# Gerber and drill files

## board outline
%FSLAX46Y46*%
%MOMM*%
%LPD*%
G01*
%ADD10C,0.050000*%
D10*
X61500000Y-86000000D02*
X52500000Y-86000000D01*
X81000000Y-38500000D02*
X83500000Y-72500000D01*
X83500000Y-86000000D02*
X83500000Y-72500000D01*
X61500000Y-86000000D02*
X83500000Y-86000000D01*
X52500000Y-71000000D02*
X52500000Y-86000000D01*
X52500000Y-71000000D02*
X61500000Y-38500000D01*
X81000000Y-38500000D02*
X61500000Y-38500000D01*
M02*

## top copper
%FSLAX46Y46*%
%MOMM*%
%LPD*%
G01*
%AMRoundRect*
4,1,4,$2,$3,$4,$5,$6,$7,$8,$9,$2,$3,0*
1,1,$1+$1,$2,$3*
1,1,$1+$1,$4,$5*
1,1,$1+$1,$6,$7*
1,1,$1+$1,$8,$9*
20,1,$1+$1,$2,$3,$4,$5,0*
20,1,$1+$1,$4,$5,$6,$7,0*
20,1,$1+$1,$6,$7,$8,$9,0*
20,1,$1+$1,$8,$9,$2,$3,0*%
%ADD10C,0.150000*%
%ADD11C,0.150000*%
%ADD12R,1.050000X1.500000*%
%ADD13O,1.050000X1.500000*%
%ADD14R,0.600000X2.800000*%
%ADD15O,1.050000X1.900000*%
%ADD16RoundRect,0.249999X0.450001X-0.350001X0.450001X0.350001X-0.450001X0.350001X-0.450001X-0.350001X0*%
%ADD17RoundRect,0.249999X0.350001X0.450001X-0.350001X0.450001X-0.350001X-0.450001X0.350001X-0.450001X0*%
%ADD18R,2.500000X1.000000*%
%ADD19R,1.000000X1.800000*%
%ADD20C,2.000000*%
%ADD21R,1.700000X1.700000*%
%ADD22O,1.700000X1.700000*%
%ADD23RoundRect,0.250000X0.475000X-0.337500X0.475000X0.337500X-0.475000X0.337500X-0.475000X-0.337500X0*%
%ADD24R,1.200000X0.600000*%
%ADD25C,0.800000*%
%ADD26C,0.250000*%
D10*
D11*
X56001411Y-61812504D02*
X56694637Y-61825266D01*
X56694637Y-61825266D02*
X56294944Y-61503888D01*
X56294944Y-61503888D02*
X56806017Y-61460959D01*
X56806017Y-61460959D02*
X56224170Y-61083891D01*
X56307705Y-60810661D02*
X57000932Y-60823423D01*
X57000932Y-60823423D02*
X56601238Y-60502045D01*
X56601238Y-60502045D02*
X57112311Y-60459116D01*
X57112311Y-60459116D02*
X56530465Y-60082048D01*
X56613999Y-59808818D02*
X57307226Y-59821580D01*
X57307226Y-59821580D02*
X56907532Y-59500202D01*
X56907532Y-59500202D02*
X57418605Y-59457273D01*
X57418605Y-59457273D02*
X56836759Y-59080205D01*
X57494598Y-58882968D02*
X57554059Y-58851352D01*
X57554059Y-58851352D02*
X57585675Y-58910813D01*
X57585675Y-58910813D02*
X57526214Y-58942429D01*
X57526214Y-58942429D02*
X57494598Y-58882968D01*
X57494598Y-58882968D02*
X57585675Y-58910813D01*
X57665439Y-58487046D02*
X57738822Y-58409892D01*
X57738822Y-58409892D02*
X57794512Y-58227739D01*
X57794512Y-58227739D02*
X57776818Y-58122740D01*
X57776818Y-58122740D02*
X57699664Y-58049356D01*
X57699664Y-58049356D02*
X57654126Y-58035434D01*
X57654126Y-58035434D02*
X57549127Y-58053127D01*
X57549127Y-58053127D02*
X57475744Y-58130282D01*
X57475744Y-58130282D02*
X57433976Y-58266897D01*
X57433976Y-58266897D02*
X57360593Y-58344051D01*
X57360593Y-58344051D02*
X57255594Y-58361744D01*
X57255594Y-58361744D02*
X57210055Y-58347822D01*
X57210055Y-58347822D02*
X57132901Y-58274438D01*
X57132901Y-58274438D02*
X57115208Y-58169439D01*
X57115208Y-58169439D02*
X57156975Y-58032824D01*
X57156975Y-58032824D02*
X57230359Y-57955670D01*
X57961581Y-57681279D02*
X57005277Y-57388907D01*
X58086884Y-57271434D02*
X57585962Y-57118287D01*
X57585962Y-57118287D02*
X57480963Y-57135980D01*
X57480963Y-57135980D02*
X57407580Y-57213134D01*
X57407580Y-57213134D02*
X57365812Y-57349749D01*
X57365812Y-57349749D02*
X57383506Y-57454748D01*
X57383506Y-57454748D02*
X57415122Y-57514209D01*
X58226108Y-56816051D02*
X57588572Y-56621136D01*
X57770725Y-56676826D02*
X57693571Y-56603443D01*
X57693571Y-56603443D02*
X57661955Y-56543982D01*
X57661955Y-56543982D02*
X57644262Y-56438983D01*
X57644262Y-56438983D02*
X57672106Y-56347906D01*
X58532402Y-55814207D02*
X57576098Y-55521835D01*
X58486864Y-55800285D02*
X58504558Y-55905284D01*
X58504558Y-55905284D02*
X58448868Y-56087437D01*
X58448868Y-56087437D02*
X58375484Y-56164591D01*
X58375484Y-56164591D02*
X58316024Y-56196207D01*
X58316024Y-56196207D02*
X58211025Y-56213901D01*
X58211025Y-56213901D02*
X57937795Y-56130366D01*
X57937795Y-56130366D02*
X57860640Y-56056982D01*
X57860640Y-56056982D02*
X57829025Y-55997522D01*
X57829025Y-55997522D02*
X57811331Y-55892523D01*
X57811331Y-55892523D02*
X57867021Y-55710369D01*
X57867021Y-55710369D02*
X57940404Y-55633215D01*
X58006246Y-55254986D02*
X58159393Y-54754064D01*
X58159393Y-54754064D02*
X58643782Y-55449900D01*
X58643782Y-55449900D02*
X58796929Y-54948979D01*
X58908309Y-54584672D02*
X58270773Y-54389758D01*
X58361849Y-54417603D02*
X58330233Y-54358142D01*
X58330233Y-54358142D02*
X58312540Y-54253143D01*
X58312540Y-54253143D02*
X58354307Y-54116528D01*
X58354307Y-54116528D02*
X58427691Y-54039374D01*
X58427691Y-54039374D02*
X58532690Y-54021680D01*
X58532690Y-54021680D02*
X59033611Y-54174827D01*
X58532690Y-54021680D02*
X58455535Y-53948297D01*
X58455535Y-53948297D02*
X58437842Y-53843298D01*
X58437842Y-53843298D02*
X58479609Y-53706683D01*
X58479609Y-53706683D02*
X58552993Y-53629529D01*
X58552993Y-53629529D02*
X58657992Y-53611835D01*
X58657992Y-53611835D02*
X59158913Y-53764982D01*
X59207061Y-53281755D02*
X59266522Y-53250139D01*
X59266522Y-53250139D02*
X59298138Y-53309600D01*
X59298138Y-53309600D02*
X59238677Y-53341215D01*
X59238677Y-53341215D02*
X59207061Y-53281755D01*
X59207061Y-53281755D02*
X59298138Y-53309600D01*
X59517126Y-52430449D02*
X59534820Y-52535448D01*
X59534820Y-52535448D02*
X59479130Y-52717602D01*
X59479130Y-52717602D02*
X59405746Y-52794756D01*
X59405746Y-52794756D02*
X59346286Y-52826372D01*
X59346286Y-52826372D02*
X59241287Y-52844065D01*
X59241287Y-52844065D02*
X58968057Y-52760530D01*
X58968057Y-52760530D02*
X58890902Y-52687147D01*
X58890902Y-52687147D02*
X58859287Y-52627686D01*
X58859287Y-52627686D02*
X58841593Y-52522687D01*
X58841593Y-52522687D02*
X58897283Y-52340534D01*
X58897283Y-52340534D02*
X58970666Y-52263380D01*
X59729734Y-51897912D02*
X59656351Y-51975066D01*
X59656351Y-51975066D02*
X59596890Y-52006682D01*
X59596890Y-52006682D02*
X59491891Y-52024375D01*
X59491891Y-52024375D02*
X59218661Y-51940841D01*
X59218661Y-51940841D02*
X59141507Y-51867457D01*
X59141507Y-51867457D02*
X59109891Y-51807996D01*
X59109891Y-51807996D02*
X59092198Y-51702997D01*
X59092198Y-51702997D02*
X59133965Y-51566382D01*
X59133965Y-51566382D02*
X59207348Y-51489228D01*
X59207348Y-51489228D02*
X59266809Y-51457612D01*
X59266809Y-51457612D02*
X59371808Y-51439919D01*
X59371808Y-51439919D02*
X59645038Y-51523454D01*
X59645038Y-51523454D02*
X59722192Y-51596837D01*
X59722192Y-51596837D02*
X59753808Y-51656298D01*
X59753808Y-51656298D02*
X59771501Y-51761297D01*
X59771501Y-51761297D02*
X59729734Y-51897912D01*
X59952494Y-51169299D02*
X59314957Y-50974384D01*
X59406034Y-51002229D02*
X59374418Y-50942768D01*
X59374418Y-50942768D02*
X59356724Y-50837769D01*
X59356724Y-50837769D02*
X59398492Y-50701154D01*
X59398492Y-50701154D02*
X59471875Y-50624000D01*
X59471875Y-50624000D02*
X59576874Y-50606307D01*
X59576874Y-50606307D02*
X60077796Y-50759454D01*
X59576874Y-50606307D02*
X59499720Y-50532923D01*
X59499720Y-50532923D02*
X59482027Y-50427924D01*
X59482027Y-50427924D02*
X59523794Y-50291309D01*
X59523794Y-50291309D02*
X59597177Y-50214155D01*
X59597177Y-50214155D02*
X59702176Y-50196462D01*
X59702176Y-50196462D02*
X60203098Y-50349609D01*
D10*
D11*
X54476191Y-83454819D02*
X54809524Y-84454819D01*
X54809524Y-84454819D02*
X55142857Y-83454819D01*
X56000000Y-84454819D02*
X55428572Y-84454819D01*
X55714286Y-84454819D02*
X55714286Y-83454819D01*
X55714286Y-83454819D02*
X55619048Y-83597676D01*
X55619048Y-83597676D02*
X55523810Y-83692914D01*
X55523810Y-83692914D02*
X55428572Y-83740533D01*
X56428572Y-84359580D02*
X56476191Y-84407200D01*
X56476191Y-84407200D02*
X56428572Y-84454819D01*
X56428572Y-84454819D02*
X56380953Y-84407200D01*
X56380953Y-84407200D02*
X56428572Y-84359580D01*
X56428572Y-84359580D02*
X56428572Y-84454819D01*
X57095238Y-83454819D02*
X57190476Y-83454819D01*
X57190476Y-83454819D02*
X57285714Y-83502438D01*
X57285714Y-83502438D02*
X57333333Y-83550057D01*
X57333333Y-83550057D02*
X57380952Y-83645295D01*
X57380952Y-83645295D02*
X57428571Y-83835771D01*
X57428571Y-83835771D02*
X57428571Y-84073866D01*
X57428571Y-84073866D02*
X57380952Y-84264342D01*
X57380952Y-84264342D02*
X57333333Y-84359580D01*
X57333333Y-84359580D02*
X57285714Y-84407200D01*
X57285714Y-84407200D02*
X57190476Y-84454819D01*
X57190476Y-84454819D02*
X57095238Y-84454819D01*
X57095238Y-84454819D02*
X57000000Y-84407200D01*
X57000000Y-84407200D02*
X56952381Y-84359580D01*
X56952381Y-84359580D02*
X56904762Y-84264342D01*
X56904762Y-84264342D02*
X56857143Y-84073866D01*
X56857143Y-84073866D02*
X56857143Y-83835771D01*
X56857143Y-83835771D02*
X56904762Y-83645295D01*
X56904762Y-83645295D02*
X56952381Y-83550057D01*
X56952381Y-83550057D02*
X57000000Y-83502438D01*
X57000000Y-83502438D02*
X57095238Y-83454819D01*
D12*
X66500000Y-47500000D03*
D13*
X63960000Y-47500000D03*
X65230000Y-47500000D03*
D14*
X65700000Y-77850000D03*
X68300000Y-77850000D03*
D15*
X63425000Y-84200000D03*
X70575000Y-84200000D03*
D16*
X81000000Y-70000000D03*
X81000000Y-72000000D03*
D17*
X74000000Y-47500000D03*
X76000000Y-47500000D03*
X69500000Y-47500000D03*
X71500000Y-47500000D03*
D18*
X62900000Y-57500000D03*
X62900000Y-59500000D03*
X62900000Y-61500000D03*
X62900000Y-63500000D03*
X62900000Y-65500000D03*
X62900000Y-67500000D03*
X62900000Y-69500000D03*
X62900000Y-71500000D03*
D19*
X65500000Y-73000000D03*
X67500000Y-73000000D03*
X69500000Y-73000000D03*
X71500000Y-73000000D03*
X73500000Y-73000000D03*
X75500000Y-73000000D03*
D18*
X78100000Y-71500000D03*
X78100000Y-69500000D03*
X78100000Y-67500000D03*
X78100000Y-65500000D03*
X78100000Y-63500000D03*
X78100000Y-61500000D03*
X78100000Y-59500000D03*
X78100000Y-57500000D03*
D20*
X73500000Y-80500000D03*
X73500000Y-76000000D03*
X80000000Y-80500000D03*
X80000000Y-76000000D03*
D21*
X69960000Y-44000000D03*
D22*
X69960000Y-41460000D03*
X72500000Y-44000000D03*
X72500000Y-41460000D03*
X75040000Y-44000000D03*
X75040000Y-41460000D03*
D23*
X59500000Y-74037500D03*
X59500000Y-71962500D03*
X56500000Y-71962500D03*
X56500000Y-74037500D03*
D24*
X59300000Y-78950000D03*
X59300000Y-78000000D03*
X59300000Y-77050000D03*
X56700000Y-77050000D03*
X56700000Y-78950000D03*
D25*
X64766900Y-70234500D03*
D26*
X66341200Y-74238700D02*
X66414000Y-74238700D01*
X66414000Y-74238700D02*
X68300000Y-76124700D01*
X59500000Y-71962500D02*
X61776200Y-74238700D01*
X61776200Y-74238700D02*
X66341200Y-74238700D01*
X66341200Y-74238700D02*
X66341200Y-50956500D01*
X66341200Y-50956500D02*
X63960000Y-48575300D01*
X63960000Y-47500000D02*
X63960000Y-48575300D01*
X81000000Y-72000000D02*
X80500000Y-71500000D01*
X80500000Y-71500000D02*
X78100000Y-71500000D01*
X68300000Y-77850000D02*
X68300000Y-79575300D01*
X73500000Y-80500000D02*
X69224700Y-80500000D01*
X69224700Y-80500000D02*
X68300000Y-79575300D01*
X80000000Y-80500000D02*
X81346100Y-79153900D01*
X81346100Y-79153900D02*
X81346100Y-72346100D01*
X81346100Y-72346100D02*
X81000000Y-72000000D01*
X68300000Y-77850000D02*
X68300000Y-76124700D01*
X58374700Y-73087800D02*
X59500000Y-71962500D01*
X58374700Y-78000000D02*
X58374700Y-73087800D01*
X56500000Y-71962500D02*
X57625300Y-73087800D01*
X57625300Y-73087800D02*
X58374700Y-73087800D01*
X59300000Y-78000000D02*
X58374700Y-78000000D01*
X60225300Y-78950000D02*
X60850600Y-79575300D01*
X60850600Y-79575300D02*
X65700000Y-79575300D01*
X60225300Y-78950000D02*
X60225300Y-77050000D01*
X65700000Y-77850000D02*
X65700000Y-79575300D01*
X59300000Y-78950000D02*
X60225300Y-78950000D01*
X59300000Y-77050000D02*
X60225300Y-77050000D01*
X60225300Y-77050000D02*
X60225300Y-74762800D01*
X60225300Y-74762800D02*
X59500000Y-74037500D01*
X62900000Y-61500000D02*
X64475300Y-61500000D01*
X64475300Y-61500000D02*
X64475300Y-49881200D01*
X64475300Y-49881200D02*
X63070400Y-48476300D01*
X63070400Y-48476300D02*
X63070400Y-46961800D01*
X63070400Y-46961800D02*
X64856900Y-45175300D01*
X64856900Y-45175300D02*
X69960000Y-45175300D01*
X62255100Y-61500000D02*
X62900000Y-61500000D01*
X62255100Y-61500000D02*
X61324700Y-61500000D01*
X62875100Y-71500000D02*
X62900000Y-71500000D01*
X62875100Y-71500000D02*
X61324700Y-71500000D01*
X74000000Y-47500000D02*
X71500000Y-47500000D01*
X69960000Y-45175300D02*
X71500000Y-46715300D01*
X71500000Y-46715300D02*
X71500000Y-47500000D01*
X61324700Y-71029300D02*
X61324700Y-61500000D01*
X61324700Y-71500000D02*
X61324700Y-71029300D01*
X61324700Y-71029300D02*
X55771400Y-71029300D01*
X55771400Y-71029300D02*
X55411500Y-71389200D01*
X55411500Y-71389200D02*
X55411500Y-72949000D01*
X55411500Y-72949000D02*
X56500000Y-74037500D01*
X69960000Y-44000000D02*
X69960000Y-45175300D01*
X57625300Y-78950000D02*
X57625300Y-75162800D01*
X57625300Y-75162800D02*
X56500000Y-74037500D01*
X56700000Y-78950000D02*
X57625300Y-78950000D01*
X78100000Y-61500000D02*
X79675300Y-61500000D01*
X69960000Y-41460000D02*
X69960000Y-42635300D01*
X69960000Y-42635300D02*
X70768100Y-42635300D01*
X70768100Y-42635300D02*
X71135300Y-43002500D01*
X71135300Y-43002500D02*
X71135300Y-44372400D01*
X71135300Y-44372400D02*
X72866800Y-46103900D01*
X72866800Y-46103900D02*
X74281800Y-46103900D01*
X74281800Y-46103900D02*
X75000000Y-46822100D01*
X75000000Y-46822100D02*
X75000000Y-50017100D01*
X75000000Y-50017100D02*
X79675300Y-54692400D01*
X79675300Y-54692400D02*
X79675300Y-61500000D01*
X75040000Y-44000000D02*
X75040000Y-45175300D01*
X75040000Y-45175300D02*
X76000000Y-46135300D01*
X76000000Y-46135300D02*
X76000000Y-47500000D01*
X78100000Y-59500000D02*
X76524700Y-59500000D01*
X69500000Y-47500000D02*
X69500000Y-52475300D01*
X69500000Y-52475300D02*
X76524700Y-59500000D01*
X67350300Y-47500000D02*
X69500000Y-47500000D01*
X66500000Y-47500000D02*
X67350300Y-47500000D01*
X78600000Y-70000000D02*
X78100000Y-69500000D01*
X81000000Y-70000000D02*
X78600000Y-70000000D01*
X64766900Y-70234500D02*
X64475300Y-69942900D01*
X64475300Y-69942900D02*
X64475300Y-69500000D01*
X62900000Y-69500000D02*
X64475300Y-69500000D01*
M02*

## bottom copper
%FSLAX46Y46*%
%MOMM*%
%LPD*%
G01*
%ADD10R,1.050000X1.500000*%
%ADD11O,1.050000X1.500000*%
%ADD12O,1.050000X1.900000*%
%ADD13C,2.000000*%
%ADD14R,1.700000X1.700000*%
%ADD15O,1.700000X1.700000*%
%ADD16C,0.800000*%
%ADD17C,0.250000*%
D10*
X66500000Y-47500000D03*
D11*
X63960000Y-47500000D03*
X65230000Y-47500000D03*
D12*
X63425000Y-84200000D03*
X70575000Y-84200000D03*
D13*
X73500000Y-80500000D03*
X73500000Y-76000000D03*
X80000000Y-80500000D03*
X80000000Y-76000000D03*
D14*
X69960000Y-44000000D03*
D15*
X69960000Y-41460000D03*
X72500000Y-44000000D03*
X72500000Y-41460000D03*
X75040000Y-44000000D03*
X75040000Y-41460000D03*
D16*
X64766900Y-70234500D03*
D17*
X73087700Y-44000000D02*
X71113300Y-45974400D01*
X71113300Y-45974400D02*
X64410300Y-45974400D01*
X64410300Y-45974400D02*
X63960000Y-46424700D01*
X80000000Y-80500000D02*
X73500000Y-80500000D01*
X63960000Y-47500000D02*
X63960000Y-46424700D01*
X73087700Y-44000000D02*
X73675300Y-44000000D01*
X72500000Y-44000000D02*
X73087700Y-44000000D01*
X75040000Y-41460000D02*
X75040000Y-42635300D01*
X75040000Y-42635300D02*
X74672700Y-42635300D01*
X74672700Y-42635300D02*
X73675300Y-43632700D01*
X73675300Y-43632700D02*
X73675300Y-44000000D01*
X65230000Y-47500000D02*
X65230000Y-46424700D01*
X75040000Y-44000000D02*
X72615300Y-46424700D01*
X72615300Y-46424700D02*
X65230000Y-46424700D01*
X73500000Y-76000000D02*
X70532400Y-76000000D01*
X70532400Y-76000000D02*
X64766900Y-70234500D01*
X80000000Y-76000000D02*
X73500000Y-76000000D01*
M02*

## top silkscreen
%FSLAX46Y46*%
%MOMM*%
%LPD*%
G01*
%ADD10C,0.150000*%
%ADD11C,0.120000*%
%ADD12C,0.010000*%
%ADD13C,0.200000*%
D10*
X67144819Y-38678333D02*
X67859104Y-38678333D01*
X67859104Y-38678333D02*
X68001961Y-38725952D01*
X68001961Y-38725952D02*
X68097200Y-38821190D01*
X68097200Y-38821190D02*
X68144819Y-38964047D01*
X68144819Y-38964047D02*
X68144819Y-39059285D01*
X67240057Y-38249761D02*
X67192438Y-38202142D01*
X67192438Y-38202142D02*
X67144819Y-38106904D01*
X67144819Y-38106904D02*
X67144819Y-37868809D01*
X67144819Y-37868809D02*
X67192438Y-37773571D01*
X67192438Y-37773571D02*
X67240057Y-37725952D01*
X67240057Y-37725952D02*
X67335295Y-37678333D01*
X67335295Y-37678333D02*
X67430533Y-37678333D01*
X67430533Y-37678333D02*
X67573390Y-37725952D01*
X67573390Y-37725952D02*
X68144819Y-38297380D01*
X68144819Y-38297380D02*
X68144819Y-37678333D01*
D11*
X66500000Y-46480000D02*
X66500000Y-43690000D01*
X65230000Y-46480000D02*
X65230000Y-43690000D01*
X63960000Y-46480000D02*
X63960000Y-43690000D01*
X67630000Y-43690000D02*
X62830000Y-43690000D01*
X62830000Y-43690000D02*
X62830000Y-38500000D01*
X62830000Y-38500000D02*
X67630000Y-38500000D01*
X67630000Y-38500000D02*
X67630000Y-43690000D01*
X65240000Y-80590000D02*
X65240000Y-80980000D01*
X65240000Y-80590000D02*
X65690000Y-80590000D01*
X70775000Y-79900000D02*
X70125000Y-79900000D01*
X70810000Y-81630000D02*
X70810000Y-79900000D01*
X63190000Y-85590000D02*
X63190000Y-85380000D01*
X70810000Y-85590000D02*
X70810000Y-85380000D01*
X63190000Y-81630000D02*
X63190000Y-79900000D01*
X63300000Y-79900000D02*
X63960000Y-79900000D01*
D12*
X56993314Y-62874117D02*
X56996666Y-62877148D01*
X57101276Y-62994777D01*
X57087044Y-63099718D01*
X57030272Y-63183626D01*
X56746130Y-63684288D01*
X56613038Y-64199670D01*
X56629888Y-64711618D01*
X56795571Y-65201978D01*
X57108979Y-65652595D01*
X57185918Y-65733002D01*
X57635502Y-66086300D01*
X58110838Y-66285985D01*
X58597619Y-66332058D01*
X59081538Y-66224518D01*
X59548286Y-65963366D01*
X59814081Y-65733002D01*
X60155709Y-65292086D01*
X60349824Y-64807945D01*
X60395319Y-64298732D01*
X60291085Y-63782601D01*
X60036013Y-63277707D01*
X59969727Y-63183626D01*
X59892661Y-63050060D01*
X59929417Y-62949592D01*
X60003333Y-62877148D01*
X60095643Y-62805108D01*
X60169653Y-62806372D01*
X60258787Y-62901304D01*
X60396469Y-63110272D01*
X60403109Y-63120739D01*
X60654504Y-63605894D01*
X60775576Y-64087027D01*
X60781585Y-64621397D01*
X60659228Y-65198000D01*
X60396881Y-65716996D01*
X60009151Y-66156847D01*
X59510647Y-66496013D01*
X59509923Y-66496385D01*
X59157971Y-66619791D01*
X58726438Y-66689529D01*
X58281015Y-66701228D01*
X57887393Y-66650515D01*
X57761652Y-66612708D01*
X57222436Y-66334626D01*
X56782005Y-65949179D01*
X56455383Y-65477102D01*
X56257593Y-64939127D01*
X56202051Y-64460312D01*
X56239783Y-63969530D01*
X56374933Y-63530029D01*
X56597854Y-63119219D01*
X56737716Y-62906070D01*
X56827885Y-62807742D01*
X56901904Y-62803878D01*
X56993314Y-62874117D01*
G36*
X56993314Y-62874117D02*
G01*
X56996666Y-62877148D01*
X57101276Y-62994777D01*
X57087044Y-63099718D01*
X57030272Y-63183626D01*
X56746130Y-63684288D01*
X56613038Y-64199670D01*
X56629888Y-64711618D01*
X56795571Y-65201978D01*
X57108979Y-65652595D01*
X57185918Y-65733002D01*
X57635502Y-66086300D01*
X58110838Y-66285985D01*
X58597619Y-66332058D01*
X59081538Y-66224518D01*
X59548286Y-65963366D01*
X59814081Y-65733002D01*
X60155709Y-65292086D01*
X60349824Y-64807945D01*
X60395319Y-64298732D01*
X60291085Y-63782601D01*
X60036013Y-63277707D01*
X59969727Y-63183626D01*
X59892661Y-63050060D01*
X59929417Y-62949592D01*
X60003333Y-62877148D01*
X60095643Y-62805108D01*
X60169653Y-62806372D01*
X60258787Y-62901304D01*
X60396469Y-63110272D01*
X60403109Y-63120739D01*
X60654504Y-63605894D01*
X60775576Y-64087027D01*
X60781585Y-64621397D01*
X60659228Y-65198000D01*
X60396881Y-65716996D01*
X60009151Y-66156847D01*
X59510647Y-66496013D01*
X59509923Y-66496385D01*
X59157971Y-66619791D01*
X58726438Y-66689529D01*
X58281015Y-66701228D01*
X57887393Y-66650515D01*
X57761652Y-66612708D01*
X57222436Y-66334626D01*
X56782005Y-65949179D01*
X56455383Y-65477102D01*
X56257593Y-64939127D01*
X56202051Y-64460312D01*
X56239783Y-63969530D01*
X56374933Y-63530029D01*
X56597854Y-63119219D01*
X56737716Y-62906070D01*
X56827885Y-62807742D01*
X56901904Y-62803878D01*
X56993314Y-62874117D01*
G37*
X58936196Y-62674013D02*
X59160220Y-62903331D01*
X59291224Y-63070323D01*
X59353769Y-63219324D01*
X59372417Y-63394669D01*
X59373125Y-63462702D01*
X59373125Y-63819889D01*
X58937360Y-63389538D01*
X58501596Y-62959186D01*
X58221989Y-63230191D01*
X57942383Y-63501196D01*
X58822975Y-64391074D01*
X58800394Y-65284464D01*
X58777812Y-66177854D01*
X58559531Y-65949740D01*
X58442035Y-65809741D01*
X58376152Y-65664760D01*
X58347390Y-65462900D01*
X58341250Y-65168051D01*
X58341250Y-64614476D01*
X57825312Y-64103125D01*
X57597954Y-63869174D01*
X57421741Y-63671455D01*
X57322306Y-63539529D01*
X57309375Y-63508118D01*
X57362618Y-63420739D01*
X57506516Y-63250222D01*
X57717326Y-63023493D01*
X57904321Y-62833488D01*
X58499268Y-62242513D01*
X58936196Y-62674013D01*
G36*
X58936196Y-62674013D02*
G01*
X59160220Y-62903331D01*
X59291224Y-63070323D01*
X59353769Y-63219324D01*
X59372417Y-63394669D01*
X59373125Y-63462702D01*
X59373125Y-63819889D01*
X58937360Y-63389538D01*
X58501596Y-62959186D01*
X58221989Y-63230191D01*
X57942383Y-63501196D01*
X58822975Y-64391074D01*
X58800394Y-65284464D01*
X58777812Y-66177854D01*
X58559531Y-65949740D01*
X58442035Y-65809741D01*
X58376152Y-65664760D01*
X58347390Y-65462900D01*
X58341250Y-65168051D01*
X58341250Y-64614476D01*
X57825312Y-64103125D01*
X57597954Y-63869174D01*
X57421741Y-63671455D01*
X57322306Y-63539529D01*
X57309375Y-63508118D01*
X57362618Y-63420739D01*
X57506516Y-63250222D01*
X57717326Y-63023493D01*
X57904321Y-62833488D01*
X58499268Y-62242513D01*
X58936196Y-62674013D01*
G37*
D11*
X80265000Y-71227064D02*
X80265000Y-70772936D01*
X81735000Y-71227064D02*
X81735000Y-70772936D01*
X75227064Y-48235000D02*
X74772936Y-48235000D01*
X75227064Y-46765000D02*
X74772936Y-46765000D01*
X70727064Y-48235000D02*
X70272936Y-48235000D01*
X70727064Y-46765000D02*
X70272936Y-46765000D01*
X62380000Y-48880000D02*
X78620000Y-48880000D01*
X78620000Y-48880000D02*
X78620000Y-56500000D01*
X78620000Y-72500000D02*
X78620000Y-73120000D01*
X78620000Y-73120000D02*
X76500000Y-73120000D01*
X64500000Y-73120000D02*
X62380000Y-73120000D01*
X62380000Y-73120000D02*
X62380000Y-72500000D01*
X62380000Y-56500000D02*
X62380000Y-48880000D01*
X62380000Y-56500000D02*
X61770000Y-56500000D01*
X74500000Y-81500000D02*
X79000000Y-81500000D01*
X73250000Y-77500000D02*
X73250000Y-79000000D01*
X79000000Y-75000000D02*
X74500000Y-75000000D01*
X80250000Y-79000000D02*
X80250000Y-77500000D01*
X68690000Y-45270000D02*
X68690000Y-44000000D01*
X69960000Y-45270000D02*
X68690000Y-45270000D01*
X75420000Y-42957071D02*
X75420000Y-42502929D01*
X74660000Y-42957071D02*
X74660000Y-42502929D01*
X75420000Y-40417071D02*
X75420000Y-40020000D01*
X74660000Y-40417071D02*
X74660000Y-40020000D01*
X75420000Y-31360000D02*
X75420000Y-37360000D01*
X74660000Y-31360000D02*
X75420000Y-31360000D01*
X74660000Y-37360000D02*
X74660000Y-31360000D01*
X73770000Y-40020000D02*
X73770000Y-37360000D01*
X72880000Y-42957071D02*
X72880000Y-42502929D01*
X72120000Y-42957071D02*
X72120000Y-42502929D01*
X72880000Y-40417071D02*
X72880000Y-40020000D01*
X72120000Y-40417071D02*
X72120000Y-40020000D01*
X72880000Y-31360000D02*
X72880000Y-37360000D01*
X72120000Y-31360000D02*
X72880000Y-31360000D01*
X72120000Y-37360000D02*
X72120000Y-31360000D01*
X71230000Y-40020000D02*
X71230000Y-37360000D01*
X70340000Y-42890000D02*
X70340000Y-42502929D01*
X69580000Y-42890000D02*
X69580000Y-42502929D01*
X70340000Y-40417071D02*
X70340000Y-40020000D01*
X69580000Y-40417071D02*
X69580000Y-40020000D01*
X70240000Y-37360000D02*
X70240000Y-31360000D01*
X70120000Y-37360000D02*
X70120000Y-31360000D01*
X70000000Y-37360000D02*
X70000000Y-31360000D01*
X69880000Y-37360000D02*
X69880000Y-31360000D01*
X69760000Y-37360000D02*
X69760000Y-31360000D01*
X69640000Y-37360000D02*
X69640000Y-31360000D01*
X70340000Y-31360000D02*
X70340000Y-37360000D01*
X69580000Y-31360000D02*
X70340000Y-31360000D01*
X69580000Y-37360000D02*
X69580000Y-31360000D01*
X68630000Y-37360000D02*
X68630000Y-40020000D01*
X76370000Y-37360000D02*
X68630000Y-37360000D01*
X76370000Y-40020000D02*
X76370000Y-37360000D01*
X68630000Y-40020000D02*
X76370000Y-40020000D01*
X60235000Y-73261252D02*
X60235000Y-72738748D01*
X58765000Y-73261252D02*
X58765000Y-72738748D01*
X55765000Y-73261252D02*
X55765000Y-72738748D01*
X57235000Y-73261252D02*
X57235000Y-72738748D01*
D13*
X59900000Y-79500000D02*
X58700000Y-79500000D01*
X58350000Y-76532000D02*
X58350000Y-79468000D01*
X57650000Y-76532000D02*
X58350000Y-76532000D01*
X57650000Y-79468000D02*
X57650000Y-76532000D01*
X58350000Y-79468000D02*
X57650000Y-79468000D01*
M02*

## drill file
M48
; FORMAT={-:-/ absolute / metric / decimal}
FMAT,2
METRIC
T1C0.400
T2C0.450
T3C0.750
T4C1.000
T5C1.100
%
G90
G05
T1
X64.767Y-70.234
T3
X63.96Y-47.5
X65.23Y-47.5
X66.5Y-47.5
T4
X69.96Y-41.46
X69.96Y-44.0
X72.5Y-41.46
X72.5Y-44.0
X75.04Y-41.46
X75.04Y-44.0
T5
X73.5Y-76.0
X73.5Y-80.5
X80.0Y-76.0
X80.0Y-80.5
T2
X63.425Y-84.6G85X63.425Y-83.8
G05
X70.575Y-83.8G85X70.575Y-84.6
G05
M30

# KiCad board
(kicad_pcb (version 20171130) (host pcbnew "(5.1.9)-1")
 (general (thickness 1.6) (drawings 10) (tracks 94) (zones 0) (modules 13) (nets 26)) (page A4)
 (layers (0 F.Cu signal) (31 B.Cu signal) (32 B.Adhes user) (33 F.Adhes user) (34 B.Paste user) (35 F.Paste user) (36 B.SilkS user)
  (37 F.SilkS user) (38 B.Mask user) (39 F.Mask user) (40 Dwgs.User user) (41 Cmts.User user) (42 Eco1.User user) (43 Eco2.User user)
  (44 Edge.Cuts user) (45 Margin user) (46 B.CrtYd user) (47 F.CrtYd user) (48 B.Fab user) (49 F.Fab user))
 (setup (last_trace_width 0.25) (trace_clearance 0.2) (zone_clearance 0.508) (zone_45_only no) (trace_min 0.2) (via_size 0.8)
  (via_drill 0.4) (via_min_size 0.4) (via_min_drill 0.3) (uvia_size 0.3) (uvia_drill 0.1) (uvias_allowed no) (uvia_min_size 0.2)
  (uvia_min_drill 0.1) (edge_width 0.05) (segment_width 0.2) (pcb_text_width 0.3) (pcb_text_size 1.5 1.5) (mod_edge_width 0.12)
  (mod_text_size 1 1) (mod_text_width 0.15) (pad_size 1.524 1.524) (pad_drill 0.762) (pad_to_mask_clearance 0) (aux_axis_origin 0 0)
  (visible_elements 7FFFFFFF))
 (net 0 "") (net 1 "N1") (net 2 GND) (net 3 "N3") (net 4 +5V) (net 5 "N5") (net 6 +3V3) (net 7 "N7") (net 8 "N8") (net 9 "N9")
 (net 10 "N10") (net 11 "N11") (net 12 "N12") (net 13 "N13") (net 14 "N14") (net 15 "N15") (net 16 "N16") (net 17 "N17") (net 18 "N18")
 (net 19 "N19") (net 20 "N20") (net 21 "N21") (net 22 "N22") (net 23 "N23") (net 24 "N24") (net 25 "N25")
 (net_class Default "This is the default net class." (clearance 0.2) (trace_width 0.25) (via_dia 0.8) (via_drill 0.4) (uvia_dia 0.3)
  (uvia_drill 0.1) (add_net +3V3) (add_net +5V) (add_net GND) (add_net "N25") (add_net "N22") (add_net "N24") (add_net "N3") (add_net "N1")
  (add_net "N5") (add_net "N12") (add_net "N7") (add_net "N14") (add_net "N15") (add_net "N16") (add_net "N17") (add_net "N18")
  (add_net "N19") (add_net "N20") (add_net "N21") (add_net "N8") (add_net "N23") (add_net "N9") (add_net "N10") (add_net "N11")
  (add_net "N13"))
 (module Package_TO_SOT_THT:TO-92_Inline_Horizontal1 (layer F.Cu) (at 66.5 47.5 180)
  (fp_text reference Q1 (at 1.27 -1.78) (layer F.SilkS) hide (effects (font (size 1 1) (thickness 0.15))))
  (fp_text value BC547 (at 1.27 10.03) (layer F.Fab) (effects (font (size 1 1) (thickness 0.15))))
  (fp_line (start 0 1.02) (end 0 3.81) (layer F.SilkS) (width 0.12))
  (fp_line (start 1.27 1.02) (end 1.27 3.81) (layer F.SilkS) (width 0.12))
  (fp_line (start 2.54 1.02) (end 2.54 3.81) (layer F.SilkS) (width 0.12))
  (fp_line (start -1.13 3.81) (end 3.67 3.81) (layer F.SilkS) (width 0.12))
  (fp_line (start 3.67 3.81) (end 3.67 9) (layer F.SilkS) (width 0.12))
  (fp_line (start 3.67 9) (end -1.13 9) (layer F.SilkS) (width 0.12))
  (fp_line (start -1.13 9) (end -1.13 3.81) (layer F.SilkS) (width 0.12))
  (pad 1 thru_hole rect (at 0 0 180) (size 1.05 1.5) (drill 0.75) (layers *.Cu *.Mask) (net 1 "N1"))
  (pad 3 thru_hole oval (at 2.54 0 180) (size 1.05 1.5) (drill 0.75) (layers *.Cu *.Mask) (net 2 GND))
  (pad 2 thru_hole oval (at 1.27 0 180) (size 1.05 1.5) (drill 0.75) (layers *.Cu *.Mask) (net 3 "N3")))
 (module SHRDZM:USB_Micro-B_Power (layer F.Cu) (at 67 83)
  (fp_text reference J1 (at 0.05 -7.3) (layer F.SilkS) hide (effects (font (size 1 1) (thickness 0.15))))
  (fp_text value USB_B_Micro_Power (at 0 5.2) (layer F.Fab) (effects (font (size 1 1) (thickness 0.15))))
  (fp_line (start -1.76 -2.41) (end -1.76 -2.02) (layer F.SilkS) (width 0.12))
  (fp_line (start -1.76 -2.41) (end -1.31 -2.41) (layer F.SilkS) (width 0.12))
  (fp_line (start 3.775 -3.1) (end 3.125 -3.1) (layer F.SilkS) (width 0.12))
  (fp_line (start 3.81 -1.37) (end 3.81 -3.1) (layer F.SilkS) (width 0.12))
  (fp_line (start -3.81 2.59) (end -3.81 2.38) (layer F.SilkS) (width 0.12))
  (fp_line (start 3.81 2.59) (end 3.81 2.38) (layer F.SilkS) (width 0.12))
  (fp_line (start -3.81 -1.37) (end -3.81 -3.1) (layer F.SilkS) (width 0.12))
  (fp_line (start -3.7 -3.1) (end -3.04 -3.1) (layer F.SilkS) (width 0.12))
  (pad 1 smd rect (at -1.3 -5.15) (size 0.6 2.8) (layers F.Cu F.Paste F.Mask) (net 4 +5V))
  (pad 5 smd rect (at 1.3 -5.15) (size 0.6 2.8) (layers F.Cu F.Paste F.Mask) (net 2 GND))
  (pad "" thru_hole oval (at -3.575 1.2 180) (size 1.05 1.9) (drill oval 0.45 1.25) (layers *.Cu *.Mask))
  (pad "" thru_hole oval (at 3.575 1.2) (size 1.05 1.9) (drill oval 0.45 1.25) (layers *.Cu *.Mask)))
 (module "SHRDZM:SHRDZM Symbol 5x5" (layer F.Cu) (at 58.5 64.5)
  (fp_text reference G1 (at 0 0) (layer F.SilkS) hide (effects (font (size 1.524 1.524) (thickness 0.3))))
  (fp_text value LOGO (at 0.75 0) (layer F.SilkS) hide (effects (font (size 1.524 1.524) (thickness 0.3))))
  (fp_poly
   (pts (xy -1.506686 -1.625883) (xy -1.503334 -1.622852) (xy -1.398724 -1.505223) (xy -1.412956 -1.400282) (xy -1.469728 -1.316374)
    (xy -1.75387 -0.815712) (xy -1.886962 -0.30033) (xy -1.870112 0.211618) (xy -1.704429 0.701978) (xy -1.391021 1.152595)
    (xy -1.314082 1.233002) (xy -0.864498 1.5863) (xy -0.389162 1.785985) (xy 0.097619 1.832058) (xy 0.581538 1.724518)
    (xy 1.048286 1.463366) (xy 1.314081 1.233002) (xy 1.655709 0.792086) (xy 1.849824 0.307945) (xy 1.895319 -0.201268)
    (xy 1.791085 -0.717399) (xy 1.536013 -1.222293) (xy 1.469727 -1.316374) (xy 1.392661 -1.44994) (xy 1.429417 -1.550408)
    (xy 1.503333 -1.622852) (xy 1.595643 -1.694892) (xy 1.669653 -1.693628) (xy 1.758787 -1.598696) (xy 1.896469 -1.389728)
    (xy 1.903109 -1.379261) (xy 2.154504 -0.894106) (xy 2.275576 -0.412973) (xy 2.281585 0.121397) (xy 2.159228 0.698)
    (xy 1.896881 1.216996) (xy 1.509151 1.656847) (xy 1.010647 1.996013) (xy 1.009923 1.996385) (xy 0.657971 2.119791)
    (xy 0.226438 2.189529) (xy -0.218985 2.201228) (xy -0.612607 2.150515) (xy -0.738348 2.112708) (xy -1.277564 1.834626)
    (xy -1.717995 1.449179) (xy -2.044617 0.977102) (xy -2.242407 0.439127) (xy -2.297949 -0.039688) (xy -2.260217 -0.53047)
    (xy -2.125067 -0.969971) (xy -1.902146 -1.380781) (xy -1.762284 -1.59393) (xy -1.672115 -1.692258) (xy -1.598096 -1.696122)
    (xy -1.506686 -1.625883))
   (layer F.SilkS) (width 0.01))
  (fp_poly
   (pts (xy 0.436196 -1.825987) (xy 0.66022 -1.596669) (xy 0.791224 -1.429677) (xy 0.853769 -1.280676) (xy 0.872417 -1.105331)
    (xy 0.873125 -1.037298) (xy 0.873125 -0.680111) (xy 0.43736 -1.110462) (xy 0.001596 -1.540814) (xy -0.278011 -1.269809)
    (xy -0.557617 -0.998804) (xy 0.322975 -0.108926) (xy 0.300394 0.784464) (xy 0.277812 1.677854) (xy 0.059531 1.44974)
    (xy -0.057965 1.309741) (xy -0.123848 1.16476) (xy -0.15261 0.9629) (xy -0.15875 0.668051) (xy -0.15875 0.114476)
    (xy -0.674688 -0.396875) (xy -0.902046 -0.630826) (xy -1.078259 -0.828545) (xy -1.177694 -0.960471) (xy -1.190625 -0.991882)
    (xy -1.137382 -1.079261) (xy -0.993484 -1.249778) (xy -0.782674 -1.476507) (xy -0.595679 -1.666512) (xy -0.000732 -2.257487)
    (xy 0.436196 -1.825987))
   (layer F.SilkS) (width 0.01)))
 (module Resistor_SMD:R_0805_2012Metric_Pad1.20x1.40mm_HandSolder (layer F.Cu) (at 81 71 90)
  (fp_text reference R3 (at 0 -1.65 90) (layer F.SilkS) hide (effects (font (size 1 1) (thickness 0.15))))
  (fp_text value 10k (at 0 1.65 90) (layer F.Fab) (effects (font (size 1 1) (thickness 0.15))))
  (fp_line (start -0.227064 -0.735) (end 0.227064 -0.735) (layer F.SilkS) (width 0.12))
  (fp_line (start -0.227064 0.735) (end 0.227064 0.735) (layer F.SilkS) (width 0.12))
  (pad 2 smd roundrect (at 1 0 90) (size 1.2 1.4) (layers F.Cu F.Paste F.Mask) (roundrect_rratio 0.2083325) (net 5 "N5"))
  (pad 1 smd roundrect (at -1 0 90) (size 1.2 1.4) (layers F.Cu F.Paste F.Mask) (roundrect_rratio 0.2083325) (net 2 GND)))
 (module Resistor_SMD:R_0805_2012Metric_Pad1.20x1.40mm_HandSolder (layer F.Cu) (at 75 47.5 180)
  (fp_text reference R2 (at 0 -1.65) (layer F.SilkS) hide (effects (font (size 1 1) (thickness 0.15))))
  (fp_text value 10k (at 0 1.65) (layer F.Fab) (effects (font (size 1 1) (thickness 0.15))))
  (fp_line (start -0.227064 -0.735) (end 0.227064 -0.735) (layer F.SilkS) (width 0.12))
  (fp_line (start -0.227064 0.735) (end 0.227064 0.735) (layer F.SilkS) (width 0.12))
  (pad 2 smd roundrect (at 1 0 180) (size 1.2 1.4) (layers F.Cu F.Paste F.Mask) (roundrect_rratio 0.2083325) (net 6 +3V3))
  (pad 1 smd roundrect (at -1 0 180) (size 1.2 1.4) (layers F.Cu F.Paste F.Mask) (roundrect_rratio 0.2083325) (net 3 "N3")))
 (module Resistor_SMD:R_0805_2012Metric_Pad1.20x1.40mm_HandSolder (layer F.Cu) (at 70.5 47.5 180)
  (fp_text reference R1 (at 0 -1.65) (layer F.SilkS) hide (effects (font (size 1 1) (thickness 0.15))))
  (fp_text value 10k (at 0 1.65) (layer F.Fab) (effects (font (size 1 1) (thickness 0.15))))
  (fp_line (start -0.227064 -0.735) (end 0.227064 -0.735) (layer F.SilkS) (width 0.12))
  (fp_line (start -0.227064 0.735) (end 0.227064 0.735) (layer F.SilkS) (width 0.12))
  (pad 2 smd roundrect (at 1 0 180) (size 1.2 1.4) (layers F.Cu F.Paste F.Mask) (roundrect_rratio 0.2083325) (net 1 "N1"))
  (pad 1 smd roundrect (at -1 0 180) (size 1.2 1.4) (layers F.Cu F.Paste F.Mask) (roundrect_rratio 0.2083325) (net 6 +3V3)))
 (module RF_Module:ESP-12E (layer F.Cu) (at 70.5 61)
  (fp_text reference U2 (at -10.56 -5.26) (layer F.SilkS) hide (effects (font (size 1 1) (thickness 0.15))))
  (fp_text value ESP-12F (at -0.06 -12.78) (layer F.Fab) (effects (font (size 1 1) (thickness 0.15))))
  (fp_line (start -8.12 -12.12) (end 8.12 -12.12) (layer F.SilkS) (width 0.12))
  (fp_line (start 8.12 -12.12) (end 8.12 -4.5) (layer F.SilkS) (width 0.12))
  (fp_line (start 8.12 11.5) (end 8.12 12.12) (layer F.SilkS) (width 0.12))
  (fp_line (start 8.12 12.12) (end 6 12.12) (layer F.SilkS) (width 0.12))
  (fp_line (start -6 12.12) (end -8.12 12.12) (layer F.SilkS) (width 0.12))
  (fp_line (start -8.12 12.12) (end -8.12 11.5) (layer F.SilkS) (width 0.12))
  (fp_line (start -8.12 -4.5) (end -8.12 -12.12) (layer F.SilkS) (width 0.12))
  (fp_line (start -8.12 -4.5) (end -8.73 -4.5) (layer F.SilkS) (width 0.12))
  (pad 1 smd rect (at -7.6 -3.5) (size 2.5 1) (layers F.Cu F.Paste F.Mask) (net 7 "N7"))
  (pad 2 smd rect (at -7.6 -1.5) (size 2.5 1) (layers F.Cu F.Paste F.Mask) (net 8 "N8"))
  (pad 3 smd rect (at -7.6 0.5) (size 2.5 1) (layers F.Cu F.Paste F.Mask) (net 6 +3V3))
  (pad 4 smd rect (at -7.6 2.5) (size 2.5 1) (layers F.Cu F.Paste F.Mask) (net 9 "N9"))
  (pad 5 smd rect (at -7.6 4.5) (size 2.5 1) (layers F.Cu F.Paste F.Mask) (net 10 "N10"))
  (pad 6 smd rect (at -7.6 6.5) (size 2.5 1) (layers F.Cu F.Paste F.Mask) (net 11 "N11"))
  (pad 7 smd rect (at -7.6 8.5) (size 2.5 1) (layers F.Cu F.Paste F.Mask) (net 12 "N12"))
  (pad 8 smd rect (at -7.6 10.5) (size 2.5 1) (layers F.Cu F.Paste F.Mask) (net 6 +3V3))
  (pad 9 smd rect (at -5 12) (size 1 1.8) (layers F.Cu F.Paste F.Mask) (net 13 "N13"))
  (pad 10 smd rect (at -3 12) (size 1 1.8) (layers F.Cu F.Paste F.Mask) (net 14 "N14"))
  (pad 11 smd rect (at -1 12) (size 1 1.8) (layers F.Cu F.Paste F.Mask) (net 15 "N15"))
  (pad 12 smd rect (at 1 12) (size 1 1.8) (layers F.Cu F.Paste F.Mask) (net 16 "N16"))
  (pad 13 smd rect (at 3 12) (size 1 1.8) (layers F.Cu F.Paste F.Mask) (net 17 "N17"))
  (pad 14 smd rect (at 5 12) (size 1 1.8) (layers F.Cu F.Paste F.Mask) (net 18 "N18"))
  (pad 15 smd rect (at 7.6 10.5) (size 2.5 1) (layers F.Cu F.Paste F.Mask) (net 2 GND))
  (pad 16 smd rect (at 7.6 8.5) (size 2.5 1) (layers F.Cu F.Paste F.Mask) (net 5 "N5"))
  (pad 17 smd rect (at 7.6 6.5) (size 2.5 1) (layers F.Cu F.Paste F.Mask) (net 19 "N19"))
  (pad 18 smd rect (at 7.6 4.5) (size 2.5 1) (layers F.Cu F.Paste F.Mask) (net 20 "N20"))
  (pad 19 smd rect (at 7.6 2.5) (size 2.5 1) (layers F.Cu F.Paste F.Mask) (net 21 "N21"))
  (pad 20 smd rect (at 7.6 0.5) (size 2.5 1) (layers F.Cu F.Paste F.Mask) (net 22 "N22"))
  (pad 21 smd rect (at 7.6 -1.5) (size 2.5 1) (layers F.Cu F.Paste F.Mask) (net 1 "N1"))
  (pad 22 smd rect (at 7.6 -3.5) (size 2.5 1) (layers F.Cu F.Paste F.Mask) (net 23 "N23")))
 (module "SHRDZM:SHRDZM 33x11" (layer B.Cu) (at 66 65 270)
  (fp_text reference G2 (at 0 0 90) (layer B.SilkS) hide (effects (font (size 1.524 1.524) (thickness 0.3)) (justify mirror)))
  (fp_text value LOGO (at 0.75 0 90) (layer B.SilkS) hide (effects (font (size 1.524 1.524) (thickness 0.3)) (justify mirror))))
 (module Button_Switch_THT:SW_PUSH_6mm (layer F.Cu) (at 73.5 76)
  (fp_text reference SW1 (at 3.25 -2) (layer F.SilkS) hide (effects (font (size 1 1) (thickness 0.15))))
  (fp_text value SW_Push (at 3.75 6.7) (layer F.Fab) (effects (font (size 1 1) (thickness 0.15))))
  (fp_line (start 1 5.5) (end 5.5 5.5) (layer F.SilkS) (width 0.12))
  (fp_line (start -0.25 1.5) (end -0.25 3) (layer F.SilkS) (width 0.12))
  (fp_line (start 5.5 -1) (end 1 -1) (layer F.SilkS) (width 0.12))
  (fp_line (start 6.75 3) (end 6.75 1.5) (layer F.SilkS) (width 0.12))
  (pad 2 thru_hole circle (at 0 4.5 90) (size 2 2) (drill 1.1) (layers *.Cu *.Mask) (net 2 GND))
  (pad 1 thru_hole circle (at 0 0 90) (size 2 2) (drill 1.1) (layers *.Cu *.Mask) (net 12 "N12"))
  (pad 2 thru_hole circle (at 6.5 4.5 90) (size 2 2) (drill 1.1) (layers *.Cu *.Mask) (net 2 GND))
  (pad 1 thru_hole circle (at 6.5 0 90) (size 2 2) (drill 1.1) (layers *.Cu *.Mask) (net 12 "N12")))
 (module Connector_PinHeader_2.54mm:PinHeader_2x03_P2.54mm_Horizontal (layer F.Cu) (at 69.96 44 90)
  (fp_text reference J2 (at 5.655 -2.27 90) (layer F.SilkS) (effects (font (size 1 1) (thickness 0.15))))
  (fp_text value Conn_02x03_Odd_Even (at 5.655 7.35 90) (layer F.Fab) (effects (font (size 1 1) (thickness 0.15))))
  (fp_line (start -1.27 -1.27) (end 0 -1.27) (layer F.SilkS) (width 0.12))
  (fp_line (start -1.27 0) (end -1.27 -1.27) (layer F.SilkS) (width 0.12))
  (fp_line (start 1.042929 5.46) (end 1.497071 5.46) (layer F.SilkS) (width 0.12))
  (fp_line (start 1.042929 4.7) (end 1.497071 4.7) (layer F.SilkS) (width 0.12))
  (fp_line (start 3.582929 5.46) (end 3.98 5.46) (layer F.SilkS) (width 0.12))
  (fp_line (start 3.582929 4.7) (end 3.98 4.7) (layer F.SilkS) (width 0.12))
  (fp_line (start 12.64 5.46) (end 6.64 5.46) (layer F.SilkS) (width 0.12))
  (fp_line (start 12.64 4.7) (end 12.64 5.46) (layer F.SilkS) (width 0.12))
  (fp_line (start 6.64 4.7) (end 12.64 4.7) (layer F.SilkS) (width 0.12))
  (fp_line (start 3.98 3.81) (end 6.64 3.81) (layer F.SilkS) (width 0.12))
  (fp_line (start 1.042929 2.92) (end 1.497071 2.92) (layer F.SilkS) (width 0.12))
  (fp_line (start 1.042929 2.16) (end 1.497071 2.16) (layer F.SilkS) (width 0.12))
  (fp_line (start 3.582929 2.92) (end 3.98 2.92) (layer F.SilkS) (width 0.12))
  (fp_line (start 3.582929 2.16) (end 3.98 2.16) (layer F.SilkS) (width 0.12))
  (fp_line (start 12.64 2.92) (end 6.64 2.92) (layer F.SilkS) (width 0.12))
  (fp_line (start 12.64 2.16) (end 12.64 2.92) (layer F.SilkS) (width 0.12))
  (fp_line (start 6.64 2.16) (end 12.64 2.16) (layer F.SilkS) (width 0.12))
  (fp_line (start 3.98 1.27) (end 6.64 1.27) (layer F.SilkS) (width 0.12))
  (fp_line (start 1.11 0.38) (end 1.497071 0.38) (layer F.SilkS) (width 0.12))
  (fp_line (start 1.11 -0.38) (end 1.497071 -0.38) (layer F.SilkS) (width 0.12))
  (fp_line (start 3.582929 0.38) (end 3.98 0.38) (layer F.SilkS) (width 0.12))
  (fp_line (start 3.582929 -0.38) (end 3.98 -0.38) (layer F.SilkS) (width 0.12))
  (fp_line (start 6.64 0.28) (end 12.64 0.28) (layer F.SilkS) (width 0.12))
  (fp_line (start 6.64 0.16) (end 12.64 0.16) (layer F.SilkS) (width 0.12))
  (fp_line (start 6.64 0.04) (end 12.64 0.04) (layer F.SilkS) (width 0.12))
  (fp_line (start 6.64 -0.08) (end 12.64 -0.08) (layer F.SilkS) (width 0.12))
  (fp_line (start 6.64 -0.2) (end 12.64 -0.2) (layer F.SilkS) (width 0.12))
  (fp_line (start 6.64 -0.32) (end 12.64 -0.32) (layer F.SilkS) (width 0.12))
  (fp_line (start 12.64 0.38) (end 6.64 0.38) (layer F.SilkS) (width 0.12))
  (fp_line (start 12.64 -0.38) (end 12.64 0.38) (layer F.SilkS) (width 0.12))
  (fp_line (start 6.64 -0.38) (end 12.64 -0.38) (layer F.SilkS) (width 0.12))
  (fp_line (start 6.64 -1.33) (end 3.98 -1.33) (layer F.SilkS) (width 0.12))
  (fp_line (start 6.64 6.41) (end 6.64 -1.33) (layer F.SilkS) (width 0.12))
  (fp_line (start 3.98 6.41) (end 6.64 6.41) (layer F.SilkS) (width 0.12))
  (fp_line (start 3.98 -1.33) (end 3.98 6.41) (layer F.SilkS) (width 0.12))
  (pad 1 thru_hole rect (at 0 0 90) (size 1.7 1.7) (drill 1) (layers *.Cu *.Mask) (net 6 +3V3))
  (pad 2 thru_hole oval (at 2.54 0 90) (size 1.7 1.7) (drill 1) (layers *.Cu *.Mask) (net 22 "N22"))
  (pad 3 thru_hole oval (at 0 2.54 90) (size 1.7 1.7) (drill 1) (layers *.Cu *.Mask) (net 2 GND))
  (pad 4 thru_hole oval (at 2.54 2.54 90) (size 1.7 1.7) (drill 1) (layers *.Cu *.Mask) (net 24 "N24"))
  (pad 5 thru_hole oval (at 0 5.08 90) (size 1.7 1.7) (drill 1) (layers *.Cu *.Mask) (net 3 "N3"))
  (pad 6 thru_hole oval (at 2.54 5.08 90) (size 1.7 1.7) (drill 1) (layers *.Cu *.Mask) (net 2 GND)))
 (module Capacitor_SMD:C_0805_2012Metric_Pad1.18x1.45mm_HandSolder (layer F.Cu) (at 59.5 73 90)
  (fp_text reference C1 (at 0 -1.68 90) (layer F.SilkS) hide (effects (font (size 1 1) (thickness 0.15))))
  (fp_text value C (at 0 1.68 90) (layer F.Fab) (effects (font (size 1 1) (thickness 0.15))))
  (fp_line (start -0.261252 0.735) (end 0.261252 0.735) (layer F.SilkS) (width 0.12))
  (fp_line (start -0.261252 -0.735) (end 0.261252 -0.735) (layer F.SilkS) (width 0.12))
  (pad 1 smd roundrect (at -1.0375 0 90) (size 1.175 1.45) (layers F.Cu F.Paste F.Mask) (roundrect_rratio 0.212766) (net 4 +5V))
  (pad 2 smd roundrect (at 1.0375 0 90) (size 1.175 1.45) (layers F.Cu F.Paste F.Mask) (roundrect_rratio 0.212766) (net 2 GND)))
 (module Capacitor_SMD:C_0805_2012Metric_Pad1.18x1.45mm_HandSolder (layer F.Cu) (at 56.5 73 90)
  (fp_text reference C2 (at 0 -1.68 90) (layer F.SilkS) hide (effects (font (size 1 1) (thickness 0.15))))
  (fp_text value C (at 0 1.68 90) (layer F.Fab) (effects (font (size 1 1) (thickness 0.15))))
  (fp_line (start -0.261252 -0.735) (end 0.261252 -0.735) (layer F.SilkS) (width 0.12))
  (fp_line (start -0.261252 0.735) (end 0.261252 0.735) (layer F.SilkS) (width 0.12))
  (pad 2 smd roundrect (at 1.0375 0 90) (size 1.175 1.45) (layers F.Cu F.Paste F.Mask) (roundrect_rratio 0.212766) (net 2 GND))
  (pad 1 smd roundrect (at -1.0375 0 90) (size 1.175 1.45) (layers F.Cu F.Paste F.Mask) (roundrect_rratio 0.212766) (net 6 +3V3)))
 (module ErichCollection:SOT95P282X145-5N (layer F.Cu) (at 58 78 180)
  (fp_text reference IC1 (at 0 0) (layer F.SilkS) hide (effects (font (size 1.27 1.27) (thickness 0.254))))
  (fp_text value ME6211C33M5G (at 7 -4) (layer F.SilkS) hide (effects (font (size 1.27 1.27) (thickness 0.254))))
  (fp_line (start -1.9 -1.5) (end -0.7 -1.5) (layer F.SilkS) (width 0.2))
  (fp_line (start -0.35 1.468) (end -0.35 -1.468) (layer F.SilkS) (width 0.2))
  (fp_line (start 0.35 1.468) (end -0.35 1.468) (layer F.SilkS) (width 0.2))
  (fp_line (start 0.35 -1.468) (end 0.35 1.468) (layer F.SilkS) (width 0.2))
  (fp_line (start -0.35 -1.468) (end 0.35 -1.468) (layer F.SilkS) (width 0.2))
  (pad 1 smd rect (at -1.3 -0.95 270) (size 0.6 1.2) (layers F.Cu F.Paste F.Mask) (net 4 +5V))
  (pad 2 smd rect (at -1.3 0 270) (size 0.6 1.2) (layers F.Cu F.Paste F.Mask) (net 2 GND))
  (pad 3 smd rect (at -1.3 0.95 270) (size 0.6 1.2) (layers F.Cu F.Paste F.Mask) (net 4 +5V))
  (pad 4 smd rect (at 1.3 0.95 270) (size 0.6 1.2) (layers F.Cu F.Paste F.Mask) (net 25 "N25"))
  (pad 5 smd rect (at 1.3 -0.95 270) (size 0.6 1.2) (layers F.Cu F.Paste F.Mask) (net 6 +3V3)))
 (gr_line (start 61.5 86) (end 52.5 86) (layer Edge.Cuts) (width 0.05))
 (gr_line (start 81 38.5) (end 83.5 72.5) (layer Edge.Cuts) (width 0.05))
 (gr_line (start 83.5 86) (end 83.5 72.5) (layer Edge.Cuts) (width 0.05))
 (gr_line (start 61.5 86) (end 83.5 86) (layer Edge.Cuts) (width 0.05))
 (gr_line (start 52.5 71) (end 52.5 86) (layer Edge.Cuts) (width 0.05))
 (gr_line (start 52.5 71) (end 61.5 38.5) (layer Edge.Cuts) (width 0.05))
 (gr_line (start 81 38.5) (end 61.5 38.5) (layer Edge.Cuts) (width 0.05))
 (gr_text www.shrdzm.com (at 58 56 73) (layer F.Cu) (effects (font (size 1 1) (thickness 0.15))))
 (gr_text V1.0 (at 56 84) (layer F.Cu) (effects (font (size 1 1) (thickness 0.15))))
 (segment (start 66.3412 74.2387) (end 66.414 74.2387) (width 0.25) (layer F.Cu) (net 2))
 (segment (start 66.414 74.2387) (end 68.3 76.1247) (width 0.25) (layer F.Cu) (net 2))
 (segment (start 59.5 71.9625) (end 61.7762 74.2387) (width 0.25) (layer F.Cu) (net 2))
 (segment (start 61.7762 74.2387) (end 66.3412 74.2387) (width 0.25) (layer F.Cu) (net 2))
 (segment (start 66.3412 74.2387) (end 66.3412 50.9565) (width 0.25) (layer F.Cu) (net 2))
 (segment (start 66.3412 50.9565) (end 63.96 48.5753) (width 0.25) (layer F.Cu) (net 2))
 (segment (start 63.96 47.5) (end 63.96 48.5753) (width 0.25) (layer F.Cu) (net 2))
 (segment (start 81 72) (end 80.5 71.5) (width 0.25) (layer F.Cu) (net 2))
 (segment (start 80.5 71.5) (end 78.1 71.5) (width 0.25) (layer F.Cu) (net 2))
 (segment (start 68.3 77.85) (end 68.3 79.5753) (width 0.25) (layer F.Cu) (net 2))
 (segment (start 73.5 80.5) (end 69.2247 80.5) (width 0.25) (layer F.Cu) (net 2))
 (segment (start 69.2247 80.5) (end 68.3 79.5753) (width 0.25) (layer F.Cu) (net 2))
 (segment (start 73.0877 44) (end 71.1133 45.9744) (width 0.25) (layer B.Cu) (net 2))
 (segment (start 71.1133 45.9744) (end 64.4103 45.9744) (width 0.25) (layer B.Cu) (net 2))
 (segment (start 64.4103 45.9744) (end 63.96 46.4247) (width 0.25) (layer B.Cu) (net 2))
 (segment (start 80 80.5) (end 81.3461 79.1539) (width 0.25) (layer F.Cu) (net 2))
 (segment (start 81.3461 79.1539) (end 81.3461 72.3461) (width 0.25) (layer F.Cu) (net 2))
 (segment (start 81.3461 72.3461) (end 81 72) (width 0.25) (layer F.Cu) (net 2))
 (segment (start 80 80.5) (end 73.5 80.5) (width 0.25) (layer B.Cu) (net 2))
 (segment (start 63.96 47.5) (end 63.96 46.4247) (width 0.25) (layer B.Cu) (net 2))
 (segment (start 73.0877 44) (end 73.6753 44) (width 0.25) (layer B.Cu) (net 2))
 (segment (start 72.5 44) (end 73.0877 44) (width 0.25) (layer B.Cu) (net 2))
 (segment (start 75.04 41.46) (end 75.04 42.6353) (width 0.25) (layer B.Cu) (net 2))
 (segment (start 75.04 42.6353) (end 74.6727 42.6353) (width 0.25) (layer B.Cu) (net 2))
 (segment (start 74.6727 42.6353) (end 73.6753 43.6327) (width 0.25) (layer B.Cu) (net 2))
 (segment (start 73.6753 43.6327) (end 73.6753 44) (width 0.25) (layer B.Cu) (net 2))
 (segment (start 68.3 77.85) (end 68.3 76.1247) (width 0.25) (layer F.Cu) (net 2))
 (segment (start 58.3747 73.0878) (end 59.5 71.9625) (width 0.25) (layer F.Cu) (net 2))
 (segment (start 58.3747 78) (end 58.3747 73.0878) (width 0.25) (layer F.Cu) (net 2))
 (segment (start 56.5 71.9625) (end 57.6253 73.0878) (width 0.25) (layer F.Cu) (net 2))
 (segment (start 57.6253 73.0878) (end 58.3747 73.0878) (width 0.25) (layer F.Cu) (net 2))
 (segment (start 59.3 78) (end 58.3747 78) (width 0.25) (layer F.Cu) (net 2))
 (segment (start 60.2253 78.95) (end 60.8506 79.5753) (width 0.25) (layer F.Cu) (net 4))
 (segment (start 60.8506 79.5753) (end 65.7 79.5753) (width 0.25) (layer F.Cu) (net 4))
 (segment (start 60.2253 78.95) (end 60.2253 77.05) (width 0.25) (layer F.Cu) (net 4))
 (segment (start 65.7 77.85) (end 65.7 79.5753) (width 0.25) (layer F.Cu) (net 4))
 (segment (start 59.3 78.95) (end 60.2253 78.95) (width 0.25) (layer F.Cu) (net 4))
 (segment (start 59.3 77.05) (end 60.2253 77.05) (width 0.25) (layer F.Cu) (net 4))
 (segment (start 60.2253 77.05) (end 60.2253 74.7628) (width 0.25) (layer F.Cu) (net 4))
 (segment (start 60.2253 74.7628) (end 59.5 74.0375) (width 0.25) (layer F.Cu) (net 4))
 (segment (start 62.9 61.5) (end 64.4753 61.5) (width 0.25) (layer F.Cu) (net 6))
 (segment (start 64.4753 61.5) (end 64.4753 49.8812) (width 0.25) (layer F.Cu) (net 6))
 (segment (start 64.4753 49.8812) (end 63.0704 48.4763) (width 0.25) (layer F.Cu) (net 6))
 (segment (start 63.0704 48.4763) (end 63.0704 46.9618) (width 0.25) (layer F.Cu) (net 6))
 (segment (start 63.0704 46.9618) (end 64.8569 45.1753) (width 0.25) (layer F.Cu) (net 6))
 (segment (start 64.8569 45.1753) (end 69.96 45.1753) (width 0.25) (layer F.Cu) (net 6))
 (segment (start 62.2551 61.5) (end 62.9 61.5) (width 0.25) (layer F.Cu) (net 6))
 (segment (start 62.2551 61.5) (end 61.3247 61.5) (width 0.25) (layer F.Cu) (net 6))
 (segment (start 62.8751 71.5) (end 62.9 71.5) (width 0.25) (layer F.Cu) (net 6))
 (segment (start 62.8751 71.5) (end 61.3247 71.5) (width 0.25) (layer F.Cu) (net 6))
 (segment (start 74 47.5) (end 71.5 47.5) (width 0.25) (layer F.Cu) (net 6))
 (segment (start 69.96 45.1753) (end 71.5 46.7153) (width 0.25) (layer F.Cu) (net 6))
 (segment (start 71.5 46.7153) (end 71.5 47.5) (width 0.25) (layer F.Cu) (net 6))
 (segment (start 61.3247 71.0293) (end 61.3247 61.5) (width 0.25) (layer F.Cu) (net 6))
 (segment (start 61.3247 71.5) (end 61.3247 71.0293) (width 0.25) (layer F.Cu) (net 6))
 (segment (start 61.3247 71.0293) (end 55.7714 71.0293) (width 0.25) (layer F.Cu) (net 6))
 (segment (start 55.7714 71.0293) (end 55.4115 71.3892) (width 0.25) (layer F.Cu) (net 6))
 (segment (start 55.4115 71.3892) (end 55.4115 72.949) (width 0.25) (layer F.Cu) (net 6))
 (segment (start 55.4115 72.949) (end 56.5 74.0375) (width 0.25) (layer F.Cu) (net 6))
 (segment (start 69.96 44) (end 69.96 45.1753) (width 0.25) (layer F.Cu) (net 6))
 (segment (start 57.6253 78.95) (end 57.6253 75.1628) (width 0.25) (layer F.Cu) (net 6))
 (segment (start 57.6253 75.1628) (end 56.5 74.0375) (width 0.25) (layer F.Cu) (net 6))
 (segment (start 56.7 78.95) (end 57.6253 78.95) (width 0.25) (layer F.Cu) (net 6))
 (segment (start 78.1 61.5) (end 79.6753 61.5) (width 0.25) (layer F.Cu) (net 22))
 (segment (start 69.96 41.46) (end 69.96 42.6353) (width 0.25) (layer F.Cu) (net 22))
 (segment (start 69.96 42.6353) (end 70.7681 42.6353) (width 0.25) (layer F.Cu) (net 22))
 (segment (start 70.7681 42.6353) (end 71.1353 43.0025) (width 0.25) (layer F.Cu) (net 22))
 (segment (start 71.1353 43.0025) (end 71.1353 44.3724) (width 0.25) (layer F.Cu) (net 22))
 (segment (start 71.1353 44.3724) (end 72.8668 46.1039) (width 0.25) (layer F.Cu) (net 22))
 (segment (start 72.8668 46.1039) (end 74.2818 46.1039) (width 0.25) (layer F.Cu) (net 22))
 (segment (start 74.2818 46.1039) (end 75 46.8221) (width 0.25) (layer F.Cu) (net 22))
 (segment (start 75 46.8221) (end 75 50.0171) (width 0.25) (layer F.Cu) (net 22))
 (segment (start 75 50.0171) (end 79.6753 54.6924) (width 0.25) (layer F.Cu) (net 22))
 (segment (start 79.6753 54.6924) (end 79.6753 61.5) (width 0.25) (layer F.Cu) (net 22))
 (segment (start 65.23 47.5) (end 65.23 46.4247) (width 0.25) (layer B.Cu) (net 3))
 (segment (start 75.04 44) (end 72.6153 46.4247) (width 0.25) (layer B.Cu) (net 3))
 (segment (start 72.6153 46.4247) (end 65.23 46.4247) (width 0.25) (layer B.Cu) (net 3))
 (segment (start 75.04 44) (end 75.04 45.1753) (width 0.25) (layer F.Cu) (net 3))
 (segment (start 75.04 45.1753) (end 76 46.1353) (width 0.25) (layer F.Cu) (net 3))
 (segment (start 76 46.1353) (end 76 47.5) (width 0.25) (layer F.Cu) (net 3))
 (segment (start 78.1 59.5) (end 76.5247 59.5) (width 0.25) (layer F.Cu) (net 1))
 (segment (start 69.5 47.5) (end 69.5 52.4753) (width 0.25) (layer F.Cu) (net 1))
 (segment (start 69.5 52.4753) (end 76.5247 59.5) (width 0.25) (layer F.Cu) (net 1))
 (segment (start 67.3503 47.5) (end 69.5 47.5) (width 0.25) (layer F.Cu) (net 1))
 (segment (start 66.5 47.5) (end 67.3503 47.5) (width 0.25) (layer F.Cu) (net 1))
 (segment (start 78.6 70) (end 78.1 69.5) (width 0.25) (layer F.Cu) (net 5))
 (segment (start 81 70) (end 78.6 70) (width 0.25) (layer F.Cu) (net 5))
 (segment (start 64.7669 70.2345) (end 64.4753 69.9429) (width 0.25) (layer F.Cu) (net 12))
 (segment (start 64.4753 69.9429) (end 64.4753 69.5) (width 0.25) (layer F.Cu) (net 12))
 (segment (start 73.5 76) (end 70.5324 76) (width 0.25) (layer B.Cu) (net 12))
 (segment (start 70.5324 76) (end 64.7669 70.2345) (width 0.25) (layer B.Cu) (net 12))
 (segment (start 62.9 69.5) (end 64.4753 69.5) (width 0.25) (layer F.Cu) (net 12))
 (segment (start 80 76) (end 73.5 76) (width 0.25) (layer B.Cu) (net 12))
 (via (at 64.7669 70.2345) (size 0.8) (layers F.Cu B.Cu) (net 12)))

